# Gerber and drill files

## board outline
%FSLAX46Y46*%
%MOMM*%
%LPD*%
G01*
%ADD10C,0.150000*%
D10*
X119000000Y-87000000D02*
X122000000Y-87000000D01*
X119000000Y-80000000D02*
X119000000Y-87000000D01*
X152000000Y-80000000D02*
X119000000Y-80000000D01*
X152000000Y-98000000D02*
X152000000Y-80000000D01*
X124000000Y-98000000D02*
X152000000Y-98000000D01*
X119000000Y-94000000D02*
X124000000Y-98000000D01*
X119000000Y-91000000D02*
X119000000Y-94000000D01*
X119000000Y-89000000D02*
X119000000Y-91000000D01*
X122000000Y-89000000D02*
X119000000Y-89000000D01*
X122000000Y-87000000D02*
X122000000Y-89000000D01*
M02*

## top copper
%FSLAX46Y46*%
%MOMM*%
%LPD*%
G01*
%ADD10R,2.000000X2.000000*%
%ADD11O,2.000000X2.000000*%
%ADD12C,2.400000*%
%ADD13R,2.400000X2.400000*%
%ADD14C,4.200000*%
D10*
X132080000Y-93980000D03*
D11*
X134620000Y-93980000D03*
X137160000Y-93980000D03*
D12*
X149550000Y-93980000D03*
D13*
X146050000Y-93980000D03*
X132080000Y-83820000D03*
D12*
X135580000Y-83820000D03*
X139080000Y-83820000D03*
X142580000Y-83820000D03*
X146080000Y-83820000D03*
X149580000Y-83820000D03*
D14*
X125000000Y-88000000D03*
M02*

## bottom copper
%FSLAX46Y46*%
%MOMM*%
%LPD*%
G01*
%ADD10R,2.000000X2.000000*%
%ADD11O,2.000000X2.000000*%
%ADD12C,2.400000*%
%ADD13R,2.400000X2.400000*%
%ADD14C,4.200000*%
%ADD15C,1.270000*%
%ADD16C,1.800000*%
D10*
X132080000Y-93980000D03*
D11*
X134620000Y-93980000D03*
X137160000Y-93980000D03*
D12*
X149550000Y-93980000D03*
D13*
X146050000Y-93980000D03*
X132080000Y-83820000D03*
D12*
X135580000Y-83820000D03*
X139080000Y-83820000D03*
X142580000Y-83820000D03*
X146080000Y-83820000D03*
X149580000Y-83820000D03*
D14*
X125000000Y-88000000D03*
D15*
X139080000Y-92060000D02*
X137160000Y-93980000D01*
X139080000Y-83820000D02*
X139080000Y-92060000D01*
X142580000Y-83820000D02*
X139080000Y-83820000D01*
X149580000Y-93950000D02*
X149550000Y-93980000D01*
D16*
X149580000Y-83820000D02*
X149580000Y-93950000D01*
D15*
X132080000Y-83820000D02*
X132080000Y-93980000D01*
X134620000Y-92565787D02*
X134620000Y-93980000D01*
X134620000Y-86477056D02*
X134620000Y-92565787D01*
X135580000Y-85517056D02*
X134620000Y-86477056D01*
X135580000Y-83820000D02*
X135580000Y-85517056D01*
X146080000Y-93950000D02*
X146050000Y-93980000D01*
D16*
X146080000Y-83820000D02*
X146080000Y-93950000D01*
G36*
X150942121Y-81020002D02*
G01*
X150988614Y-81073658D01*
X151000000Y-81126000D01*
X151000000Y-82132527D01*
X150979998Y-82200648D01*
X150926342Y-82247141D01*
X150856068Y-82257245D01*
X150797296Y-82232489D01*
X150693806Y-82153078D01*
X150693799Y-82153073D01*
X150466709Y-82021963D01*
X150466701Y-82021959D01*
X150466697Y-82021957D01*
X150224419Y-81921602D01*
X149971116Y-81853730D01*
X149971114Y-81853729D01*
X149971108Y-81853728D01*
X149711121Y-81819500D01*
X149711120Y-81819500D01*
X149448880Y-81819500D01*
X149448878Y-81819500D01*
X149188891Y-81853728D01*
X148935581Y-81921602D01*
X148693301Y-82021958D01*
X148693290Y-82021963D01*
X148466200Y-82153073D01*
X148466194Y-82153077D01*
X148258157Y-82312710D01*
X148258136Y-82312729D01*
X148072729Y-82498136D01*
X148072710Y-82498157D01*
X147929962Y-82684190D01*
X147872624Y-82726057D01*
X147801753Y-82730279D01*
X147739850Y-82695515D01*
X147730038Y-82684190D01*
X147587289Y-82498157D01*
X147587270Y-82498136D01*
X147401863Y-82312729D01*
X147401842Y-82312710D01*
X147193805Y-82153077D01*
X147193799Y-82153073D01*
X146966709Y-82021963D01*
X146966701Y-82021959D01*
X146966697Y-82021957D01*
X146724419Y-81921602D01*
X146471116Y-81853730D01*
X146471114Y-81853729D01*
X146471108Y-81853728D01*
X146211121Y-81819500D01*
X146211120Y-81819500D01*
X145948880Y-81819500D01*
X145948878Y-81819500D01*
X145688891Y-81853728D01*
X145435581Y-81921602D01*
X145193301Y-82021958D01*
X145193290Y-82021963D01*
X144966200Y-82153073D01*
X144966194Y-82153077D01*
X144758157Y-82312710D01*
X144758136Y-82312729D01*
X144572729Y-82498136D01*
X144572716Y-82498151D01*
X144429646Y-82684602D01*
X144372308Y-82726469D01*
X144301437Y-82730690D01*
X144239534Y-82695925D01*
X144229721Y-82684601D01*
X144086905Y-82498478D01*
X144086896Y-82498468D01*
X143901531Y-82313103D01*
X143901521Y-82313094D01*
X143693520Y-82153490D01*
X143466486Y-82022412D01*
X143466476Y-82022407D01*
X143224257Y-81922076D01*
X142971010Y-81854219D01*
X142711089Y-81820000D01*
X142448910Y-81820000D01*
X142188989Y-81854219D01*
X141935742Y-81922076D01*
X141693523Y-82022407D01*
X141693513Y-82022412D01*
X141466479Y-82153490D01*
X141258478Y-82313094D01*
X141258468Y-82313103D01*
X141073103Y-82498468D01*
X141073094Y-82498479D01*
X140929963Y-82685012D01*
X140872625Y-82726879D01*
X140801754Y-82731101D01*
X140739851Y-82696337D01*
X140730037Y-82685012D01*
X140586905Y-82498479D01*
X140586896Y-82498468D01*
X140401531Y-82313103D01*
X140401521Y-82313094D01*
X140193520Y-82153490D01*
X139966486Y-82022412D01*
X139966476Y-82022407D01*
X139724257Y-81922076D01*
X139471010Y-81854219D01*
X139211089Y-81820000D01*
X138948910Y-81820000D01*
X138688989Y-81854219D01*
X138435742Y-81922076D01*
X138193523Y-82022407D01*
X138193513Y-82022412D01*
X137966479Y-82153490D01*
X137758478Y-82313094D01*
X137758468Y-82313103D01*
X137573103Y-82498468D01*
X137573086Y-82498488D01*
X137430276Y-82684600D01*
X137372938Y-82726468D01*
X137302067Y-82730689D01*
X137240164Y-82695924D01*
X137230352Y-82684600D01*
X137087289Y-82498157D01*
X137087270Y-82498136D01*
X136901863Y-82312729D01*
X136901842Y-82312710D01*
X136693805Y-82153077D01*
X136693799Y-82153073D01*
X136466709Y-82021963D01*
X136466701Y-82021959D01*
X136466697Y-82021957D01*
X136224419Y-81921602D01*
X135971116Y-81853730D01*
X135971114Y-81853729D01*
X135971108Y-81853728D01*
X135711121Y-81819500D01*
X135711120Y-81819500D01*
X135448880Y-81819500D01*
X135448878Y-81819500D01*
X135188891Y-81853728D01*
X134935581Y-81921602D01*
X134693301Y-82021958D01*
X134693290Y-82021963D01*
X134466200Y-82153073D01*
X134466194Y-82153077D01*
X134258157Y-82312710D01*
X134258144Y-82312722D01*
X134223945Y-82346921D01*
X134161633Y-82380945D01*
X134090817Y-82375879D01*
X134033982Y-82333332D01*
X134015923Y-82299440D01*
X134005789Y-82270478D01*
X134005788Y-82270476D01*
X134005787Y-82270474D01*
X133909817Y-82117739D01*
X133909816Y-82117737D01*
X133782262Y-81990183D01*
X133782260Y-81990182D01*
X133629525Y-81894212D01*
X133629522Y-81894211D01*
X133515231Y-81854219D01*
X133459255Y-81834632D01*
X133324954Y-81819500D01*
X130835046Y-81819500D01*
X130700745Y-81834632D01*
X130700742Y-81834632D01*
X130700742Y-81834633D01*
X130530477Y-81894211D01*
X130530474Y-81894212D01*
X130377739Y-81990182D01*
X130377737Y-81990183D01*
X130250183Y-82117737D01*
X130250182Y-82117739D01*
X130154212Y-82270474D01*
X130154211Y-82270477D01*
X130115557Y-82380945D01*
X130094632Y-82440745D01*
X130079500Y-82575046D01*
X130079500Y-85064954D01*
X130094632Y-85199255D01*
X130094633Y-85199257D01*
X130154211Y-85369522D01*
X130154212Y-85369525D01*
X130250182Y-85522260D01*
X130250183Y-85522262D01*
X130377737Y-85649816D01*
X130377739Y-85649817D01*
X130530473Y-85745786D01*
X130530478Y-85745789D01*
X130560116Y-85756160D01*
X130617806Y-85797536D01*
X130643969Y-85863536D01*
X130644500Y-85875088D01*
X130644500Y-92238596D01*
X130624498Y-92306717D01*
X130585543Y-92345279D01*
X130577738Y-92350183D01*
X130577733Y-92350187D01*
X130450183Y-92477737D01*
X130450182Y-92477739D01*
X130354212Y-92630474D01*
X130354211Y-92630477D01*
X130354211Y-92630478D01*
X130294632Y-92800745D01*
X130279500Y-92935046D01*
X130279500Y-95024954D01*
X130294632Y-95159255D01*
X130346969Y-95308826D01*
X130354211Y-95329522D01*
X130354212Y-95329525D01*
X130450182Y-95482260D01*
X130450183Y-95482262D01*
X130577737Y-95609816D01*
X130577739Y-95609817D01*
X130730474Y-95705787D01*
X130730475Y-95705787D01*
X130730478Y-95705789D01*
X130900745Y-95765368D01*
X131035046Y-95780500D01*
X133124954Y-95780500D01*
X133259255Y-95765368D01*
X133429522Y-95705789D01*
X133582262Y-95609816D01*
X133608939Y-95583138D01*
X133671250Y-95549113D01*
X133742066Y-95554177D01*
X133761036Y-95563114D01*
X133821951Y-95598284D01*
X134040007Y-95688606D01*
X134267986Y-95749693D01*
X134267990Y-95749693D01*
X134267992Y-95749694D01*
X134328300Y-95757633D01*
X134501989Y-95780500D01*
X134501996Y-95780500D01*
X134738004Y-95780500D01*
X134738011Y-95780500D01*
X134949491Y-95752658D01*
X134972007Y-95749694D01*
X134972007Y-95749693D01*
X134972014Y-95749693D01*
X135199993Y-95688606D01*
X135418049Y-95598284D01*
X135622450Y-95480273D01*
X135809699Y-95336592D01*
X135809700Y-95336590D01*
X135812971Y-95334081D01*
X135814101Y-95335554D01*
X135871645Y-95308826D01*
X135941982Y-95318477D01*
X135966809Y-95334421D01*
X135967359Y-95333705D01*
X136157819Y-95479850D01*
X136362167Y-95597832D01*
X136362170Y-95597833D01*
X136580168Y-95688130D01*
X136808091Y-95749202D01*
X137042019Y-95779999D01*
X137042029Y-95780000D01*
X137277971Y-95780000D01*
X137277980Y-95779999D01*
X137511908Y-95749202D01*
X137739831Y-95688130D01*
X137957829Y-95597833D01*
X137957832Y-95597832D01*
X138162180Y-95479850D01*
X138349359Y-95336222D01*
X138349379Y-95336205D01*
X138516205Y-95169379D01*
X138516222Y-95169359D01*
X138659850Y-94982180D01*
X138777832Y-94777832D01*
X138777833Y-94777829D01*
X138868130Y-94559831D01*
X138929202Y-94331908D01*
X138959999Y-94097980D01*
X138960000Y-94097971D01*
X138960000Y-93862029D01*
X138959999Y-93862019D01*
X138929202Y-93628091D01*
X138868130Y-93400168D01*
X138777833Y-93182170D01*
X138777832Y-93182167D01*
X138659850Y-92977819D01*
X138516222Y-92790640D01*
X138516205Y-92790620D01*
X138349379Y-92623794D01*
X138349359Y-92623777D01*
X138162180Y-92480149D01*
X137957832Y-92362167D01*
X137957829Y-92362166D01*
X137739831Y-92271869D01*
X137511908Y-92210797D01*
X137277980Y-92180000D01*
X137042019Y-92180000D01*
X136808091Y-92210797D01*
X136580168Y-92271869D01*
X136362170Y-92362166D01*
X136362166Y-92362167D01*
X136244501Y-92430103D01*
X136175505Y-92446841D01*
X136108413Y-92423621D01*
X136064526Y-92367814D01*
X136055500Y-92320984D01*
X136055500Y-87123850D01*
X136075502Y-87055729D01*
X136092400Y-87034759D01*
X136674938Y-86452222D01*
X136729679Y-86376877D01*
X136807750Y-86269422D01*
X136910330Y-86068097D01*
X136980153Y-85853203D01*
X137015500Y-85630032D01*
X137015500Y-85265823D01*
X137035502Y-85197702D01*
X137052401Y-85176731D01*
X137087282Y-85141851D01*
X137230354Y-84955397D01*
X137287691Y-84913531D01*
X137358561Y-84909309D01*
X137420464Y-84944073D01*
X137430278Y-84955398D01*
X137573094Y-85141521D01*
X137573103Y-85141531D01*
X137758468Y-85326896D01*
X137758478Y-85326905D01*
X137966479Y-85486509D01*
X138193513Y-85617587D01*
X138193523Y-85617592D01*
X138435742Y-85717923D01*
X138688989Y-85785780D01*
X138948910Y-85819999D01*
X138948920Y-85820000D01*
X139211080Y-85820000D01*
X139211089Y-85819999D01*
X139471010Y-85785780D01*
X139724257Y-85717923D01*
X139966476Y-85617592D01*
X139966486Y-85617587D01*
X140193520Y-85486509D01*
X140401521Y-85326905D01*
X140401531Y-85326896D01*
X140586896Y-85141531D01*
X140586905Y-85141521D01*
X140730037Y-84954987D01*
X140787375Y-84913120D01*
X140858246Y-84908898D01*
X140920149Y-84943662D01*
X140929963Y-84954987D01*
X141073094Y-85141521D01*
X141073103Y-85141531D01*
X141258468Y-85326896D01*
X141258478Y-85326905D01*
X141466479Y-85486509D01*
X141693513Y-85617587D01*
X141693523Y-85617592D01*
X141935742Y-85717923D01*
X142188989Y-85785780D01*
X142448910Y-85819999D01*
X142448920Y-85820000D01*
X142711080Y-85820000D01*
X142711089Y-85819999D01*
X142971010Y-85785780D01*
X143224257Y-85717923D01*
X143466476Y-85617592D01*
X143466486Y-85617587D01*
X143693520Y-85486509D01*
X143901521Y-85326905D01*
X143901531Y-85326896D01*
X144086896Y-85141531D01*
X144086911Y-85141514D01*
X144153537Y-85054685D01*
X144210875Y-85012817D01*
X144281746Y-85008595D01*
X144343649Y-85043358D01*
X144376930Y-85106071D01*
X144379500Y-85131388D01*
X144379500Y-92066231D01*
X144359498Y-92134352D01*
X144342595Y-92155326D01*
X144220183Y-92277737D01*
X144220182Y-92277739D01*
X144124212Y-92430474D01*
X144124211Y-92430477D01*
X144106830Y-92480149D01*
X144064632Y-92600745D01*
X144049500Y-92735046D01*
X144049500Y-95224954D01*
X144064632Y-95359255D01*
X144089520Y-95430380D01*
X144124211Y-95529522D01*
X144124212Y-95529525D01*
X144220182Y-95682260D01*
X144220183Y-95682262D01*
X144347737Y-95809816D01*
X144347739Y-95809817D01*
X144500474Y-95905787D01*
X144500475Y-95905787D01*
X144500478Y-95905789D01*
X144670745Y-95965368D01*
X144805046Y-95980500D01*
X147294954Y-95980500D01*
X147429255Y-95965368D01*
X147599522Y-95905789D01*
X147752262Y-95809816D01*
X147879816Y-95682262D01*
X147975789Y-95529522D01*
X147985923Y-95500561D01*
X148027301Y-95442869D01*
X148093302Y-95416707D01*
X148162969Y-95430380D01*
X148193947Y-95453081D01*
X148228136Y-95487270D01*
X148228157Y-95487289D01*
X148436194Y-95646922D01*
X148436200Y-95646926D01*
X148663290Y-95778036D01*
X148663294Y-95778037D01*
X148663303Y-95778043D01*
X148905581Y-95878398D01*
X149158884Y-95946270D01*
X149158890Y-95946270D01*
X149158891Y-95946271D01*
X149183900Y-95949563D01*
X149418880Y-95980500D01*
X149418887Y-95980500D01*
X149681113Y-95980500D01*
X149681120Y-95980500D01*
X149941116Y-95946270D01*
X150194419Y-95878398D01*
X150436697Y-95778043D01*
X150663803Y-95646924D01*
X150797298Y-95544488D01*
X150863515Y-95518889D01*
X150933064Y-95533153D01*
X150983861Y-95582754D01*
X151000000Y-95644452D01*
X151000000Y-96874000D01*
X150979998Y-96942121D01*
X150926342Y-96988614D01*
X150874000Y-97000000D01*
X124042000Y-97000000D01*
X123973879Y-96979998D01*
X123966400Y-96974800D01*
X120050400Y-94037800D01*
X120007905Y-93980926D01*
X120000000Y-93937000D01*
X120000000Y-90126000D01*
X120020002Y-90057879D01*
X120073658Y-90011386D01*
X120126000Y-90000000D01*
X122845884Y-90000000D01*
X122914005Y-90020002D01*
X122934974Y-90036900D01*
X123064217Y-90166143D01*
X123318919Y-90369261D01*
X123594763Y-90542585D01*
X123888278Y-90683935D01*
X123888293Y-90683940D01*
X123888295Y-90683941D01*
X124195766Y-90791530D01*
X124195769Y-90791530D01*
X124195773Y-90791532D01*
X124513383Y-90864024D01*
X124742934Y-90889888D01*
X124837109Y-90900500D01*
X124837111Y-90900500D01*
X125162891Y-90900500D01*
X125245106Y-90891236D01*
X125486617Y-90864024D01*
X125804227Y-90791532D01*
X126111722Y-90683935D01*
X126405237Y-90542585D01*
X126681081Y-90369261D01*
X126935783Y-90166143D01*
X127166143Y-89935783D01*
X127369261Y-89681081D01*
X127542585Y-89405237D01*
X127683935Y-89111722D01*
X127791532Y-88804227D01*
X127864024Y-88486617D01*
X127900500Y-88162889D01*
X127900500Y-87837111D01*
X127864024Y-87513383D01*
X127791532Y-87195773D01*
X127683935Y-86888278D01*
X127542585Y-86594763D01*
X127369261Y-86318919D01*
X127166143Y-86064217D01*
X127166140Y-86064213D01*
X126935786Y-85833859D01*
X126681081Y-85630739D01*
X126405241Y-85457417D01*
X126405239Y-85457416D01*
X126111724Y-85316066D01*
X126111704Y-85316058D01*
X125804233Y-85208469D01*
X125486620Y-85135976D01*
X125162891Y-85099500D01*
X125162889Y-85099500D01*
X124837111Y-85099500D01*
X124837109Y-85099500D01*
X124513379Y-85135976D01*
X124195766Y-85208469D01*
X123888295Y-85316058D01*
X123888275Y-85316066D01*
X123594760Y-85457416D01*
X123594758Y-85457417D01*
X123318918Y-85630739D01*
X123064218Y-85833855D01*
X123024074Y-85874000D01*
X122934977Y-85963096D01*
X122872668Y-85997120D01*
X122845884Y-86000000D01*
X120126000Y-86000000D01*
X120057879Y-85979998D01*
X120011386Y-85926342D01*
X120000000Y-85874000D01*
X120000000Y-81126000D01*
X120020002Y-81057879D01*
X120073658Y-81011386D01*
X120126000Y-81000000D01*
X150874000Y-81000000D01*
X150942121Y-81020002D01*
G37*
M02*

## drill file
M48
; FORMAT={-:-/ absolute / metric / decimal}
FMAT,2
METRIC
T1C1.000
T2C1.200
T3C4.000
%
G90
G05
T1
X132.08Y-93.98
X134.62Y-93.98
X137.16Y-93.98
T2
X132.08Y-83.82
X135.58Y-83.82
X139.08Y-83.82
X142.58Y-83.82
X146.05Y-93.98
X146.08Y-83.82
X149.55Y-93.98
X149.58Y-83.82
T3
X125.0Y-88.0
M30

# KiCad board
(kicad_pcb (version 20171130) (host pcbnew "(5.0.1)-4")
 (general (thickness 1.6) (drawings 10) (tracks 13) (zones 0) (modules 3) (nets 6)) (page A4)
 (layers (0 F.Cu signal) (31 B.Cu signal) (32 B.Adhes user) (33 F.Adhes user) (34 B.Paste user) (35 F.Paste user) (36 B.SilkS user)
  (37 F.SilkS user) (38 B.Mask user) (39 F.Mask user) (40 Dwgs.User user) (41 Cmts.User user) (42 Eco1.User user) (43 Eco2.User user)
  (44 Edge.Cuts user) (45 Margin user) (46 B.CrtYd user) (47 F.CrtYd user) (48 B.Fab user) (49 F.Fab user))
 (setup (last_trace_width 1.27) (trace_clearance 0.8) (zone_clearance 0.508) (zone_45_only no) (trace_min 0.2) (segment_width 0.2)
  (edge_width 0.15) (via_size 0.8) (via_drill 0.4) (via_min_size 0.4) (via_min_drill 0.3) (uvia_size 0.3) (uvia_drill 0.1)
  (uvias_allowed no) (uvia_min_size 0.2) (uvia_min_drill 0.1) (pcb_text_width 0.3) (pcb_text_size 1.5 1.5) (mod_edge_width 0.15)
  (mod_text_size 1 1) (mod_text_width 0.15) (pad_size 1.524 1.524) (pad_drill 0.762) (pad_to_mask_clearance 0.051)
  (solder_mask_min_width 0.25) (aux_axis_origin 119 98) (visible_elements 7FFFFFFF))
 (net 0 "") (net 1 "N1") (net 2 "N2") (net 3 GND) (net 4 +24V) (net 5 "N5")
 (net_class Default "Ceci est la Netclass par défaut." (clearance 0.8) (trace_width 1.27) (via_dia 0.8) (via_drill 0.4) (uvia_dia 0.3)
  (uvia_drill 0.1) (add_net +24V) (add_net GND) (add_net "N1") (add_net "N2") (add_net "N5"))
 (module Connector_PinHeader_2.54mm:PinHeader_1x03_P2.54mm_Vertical (layer F.Cu) (at 132.08 93.98 90)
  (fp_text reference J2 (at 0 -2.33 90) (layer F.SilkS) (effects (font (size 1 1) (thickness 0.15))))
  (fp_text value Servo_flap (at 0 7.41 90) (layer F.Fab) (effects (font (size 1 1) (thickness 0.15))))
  (pad 1 thru_hole rect (at 0 0 90) (size 2 2) (drill 1) (layers *.Cu *.Mask) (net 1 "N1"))
  (pad 2 thru_hole oval (at 0 2.54 90) (size 2 2) (drill 1) (layers *.Cu *.Mask) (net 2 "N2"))
  (pad 3 thru_hole oval (at 0 5.08 90) (size 2 2) (drill 1) (layers *.Cu *.Mask) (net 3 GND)))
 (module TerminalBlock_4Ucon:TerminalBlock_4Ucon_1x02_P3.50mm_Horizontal (layer F.Cu) (at 146.05 93.98)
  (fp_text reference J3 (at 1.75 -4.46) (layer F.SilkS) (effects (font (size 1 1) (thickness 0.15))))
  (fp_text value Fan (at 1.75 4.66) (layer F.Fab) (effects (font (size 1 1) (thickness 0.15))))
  (pad 2 thru_hole circle (at 3.5 0) (size 2.4 2.4) (drill 1.2) (layers *.Cu *.Mask) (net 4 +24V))
  (pad 1 thru_hole rect (at 0 0) (size 2.4 2.4) (drill 1.2) (layers *.Cu *.Mask) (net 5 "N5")))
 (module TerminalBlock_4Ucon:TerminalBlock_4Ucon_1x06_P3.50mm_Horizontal (layer F.Cu) (at 132.08 83.82)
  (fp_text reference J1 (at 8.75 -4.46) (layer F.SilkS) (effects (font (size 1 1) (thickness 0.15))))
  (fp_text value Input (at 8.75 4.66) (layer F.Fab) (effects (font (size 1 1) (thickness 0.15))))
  (pad 1 thru_hole rect (at 0 0) (size 2.4 2.4) (drill 1.2) (layers *.Cu *.Mask) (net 1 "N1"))
  (pad 2 thru_hole circle (at 3.5 0) (size 2.4 2.4) (drill 1.2) (layers *.Cu *.Mask) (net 2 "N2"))
  (pad 3 thru_hole circle (at 7 0) (size 2.4 2.4) (drill 1.2) (layers *.Cu *.Mask) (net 3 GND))
  (pad 4 thru_hole circle (at 10.5 0) (size 2.4 2.4) (drill 1.2) (layers *.Cu *.Mask) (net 3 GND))
  (pad 5 thru_hole circle (at 14 0) (size 2.4 2.4) (drill 1.2) (layers *.Cu *.Mask) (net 5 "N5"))
  (pad 6 thru_hole circle (at 17.5 0) (size 2.4 2.4) (drill 1.2) (layers *.Cu *.Mask) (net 4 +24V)))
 (gr_line (start 119 87) (end 122 87) (layer Edge.Cuts) (width 0.15))
 (gr_line (start 119 80) (end 119 87) (layer Edge.Cuts) (width 0.15))
 (gr_line (start 152 80) (end 119 80) (layer Edge.Cuts) (width 0.15))
 (gr_line (start 152 98) (end 152 80) (layer Edge.Cuts) (width 0.15))
 (gr_line (start 124 98) (end 152 98) (layer Edge.Cuts) (width 0.15))
 (gr_line (start 119 94) (end 124 98) (layer Edge.Cuts) (width 0.15))
 (gr_line (start 119 91) (end 119 94) (layer Edge.Cuts) (width 0.15))
 (gr_line (start 119 89) (end 119 91) (layer Edge.Cuts) (width 0.15))
 (gr_line (start 122 89) (end 119 89) (layer Edge.Cuts) (width 0.15))
 (gr_line (start 122 87) (end 122 89) (layer Edge.Cuts) (width 0.15))
 (via (at 125 88) (size 4.2) (drill 4) (layers F.Cu B.Cu) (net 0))
 (segment (start 139.08 92.06) (end 137.16 93.98) (width 1.27) (layer B.Cu) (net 3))
 (segment (start 139.08 83.82) (end 139.08 92.06) (width 1.27) (layer B.Cu) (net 3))
 (segment (start 142.58 83.82) (end 139.08 83.82) (width 1.27) (layer B.Cu) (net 3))
 (segment (start 149.58 93.95) (end 149.55 93.98) (width 1.27) (layer B.Cu) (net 4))
 (segment (start 149.58 83.82) (end 149.58 93.95) (width 1.8) (layer B.Cu) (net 4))
 (segment (start 132.08 83.82) (end 132.08 93.98) (width 1.27) (layer B.Cu) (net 1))
 (segment (start 134.62 92.565787) (end 134.62 93.98) (width 1.27) (layer B.Cu) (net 2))
 (segment (start 134.62 86.477056) (end 134.62 92.565787) (width 1.27) (layer B.Cu) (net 2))
 (segment (start 135.58 85.517056) (end 134.62 86.477056) (width 1.27) (layer B.Cu) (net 2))
 (segment (start 135.58 83.82) (end 135.58 85.517056) (width 1.27) (layer B.Cu) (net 2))
 (segment (start 146.08 93.95) (end 146.05 93.98) (width 1.27) (layer B.Cu) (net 5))
 (segment (start 146.08 83.82) (end 146.08 93.95) (width 1.8) (layer B.Cu) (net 5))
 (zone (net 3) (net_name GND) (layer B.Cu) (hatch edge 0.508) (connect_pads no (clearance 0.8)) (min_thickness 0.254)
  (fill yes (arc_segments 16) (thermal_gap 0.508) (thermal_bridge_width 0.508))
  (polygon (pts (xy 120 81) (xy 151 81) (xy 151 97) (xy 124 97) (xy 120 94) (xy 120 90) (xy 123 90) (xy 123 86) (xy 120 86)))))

